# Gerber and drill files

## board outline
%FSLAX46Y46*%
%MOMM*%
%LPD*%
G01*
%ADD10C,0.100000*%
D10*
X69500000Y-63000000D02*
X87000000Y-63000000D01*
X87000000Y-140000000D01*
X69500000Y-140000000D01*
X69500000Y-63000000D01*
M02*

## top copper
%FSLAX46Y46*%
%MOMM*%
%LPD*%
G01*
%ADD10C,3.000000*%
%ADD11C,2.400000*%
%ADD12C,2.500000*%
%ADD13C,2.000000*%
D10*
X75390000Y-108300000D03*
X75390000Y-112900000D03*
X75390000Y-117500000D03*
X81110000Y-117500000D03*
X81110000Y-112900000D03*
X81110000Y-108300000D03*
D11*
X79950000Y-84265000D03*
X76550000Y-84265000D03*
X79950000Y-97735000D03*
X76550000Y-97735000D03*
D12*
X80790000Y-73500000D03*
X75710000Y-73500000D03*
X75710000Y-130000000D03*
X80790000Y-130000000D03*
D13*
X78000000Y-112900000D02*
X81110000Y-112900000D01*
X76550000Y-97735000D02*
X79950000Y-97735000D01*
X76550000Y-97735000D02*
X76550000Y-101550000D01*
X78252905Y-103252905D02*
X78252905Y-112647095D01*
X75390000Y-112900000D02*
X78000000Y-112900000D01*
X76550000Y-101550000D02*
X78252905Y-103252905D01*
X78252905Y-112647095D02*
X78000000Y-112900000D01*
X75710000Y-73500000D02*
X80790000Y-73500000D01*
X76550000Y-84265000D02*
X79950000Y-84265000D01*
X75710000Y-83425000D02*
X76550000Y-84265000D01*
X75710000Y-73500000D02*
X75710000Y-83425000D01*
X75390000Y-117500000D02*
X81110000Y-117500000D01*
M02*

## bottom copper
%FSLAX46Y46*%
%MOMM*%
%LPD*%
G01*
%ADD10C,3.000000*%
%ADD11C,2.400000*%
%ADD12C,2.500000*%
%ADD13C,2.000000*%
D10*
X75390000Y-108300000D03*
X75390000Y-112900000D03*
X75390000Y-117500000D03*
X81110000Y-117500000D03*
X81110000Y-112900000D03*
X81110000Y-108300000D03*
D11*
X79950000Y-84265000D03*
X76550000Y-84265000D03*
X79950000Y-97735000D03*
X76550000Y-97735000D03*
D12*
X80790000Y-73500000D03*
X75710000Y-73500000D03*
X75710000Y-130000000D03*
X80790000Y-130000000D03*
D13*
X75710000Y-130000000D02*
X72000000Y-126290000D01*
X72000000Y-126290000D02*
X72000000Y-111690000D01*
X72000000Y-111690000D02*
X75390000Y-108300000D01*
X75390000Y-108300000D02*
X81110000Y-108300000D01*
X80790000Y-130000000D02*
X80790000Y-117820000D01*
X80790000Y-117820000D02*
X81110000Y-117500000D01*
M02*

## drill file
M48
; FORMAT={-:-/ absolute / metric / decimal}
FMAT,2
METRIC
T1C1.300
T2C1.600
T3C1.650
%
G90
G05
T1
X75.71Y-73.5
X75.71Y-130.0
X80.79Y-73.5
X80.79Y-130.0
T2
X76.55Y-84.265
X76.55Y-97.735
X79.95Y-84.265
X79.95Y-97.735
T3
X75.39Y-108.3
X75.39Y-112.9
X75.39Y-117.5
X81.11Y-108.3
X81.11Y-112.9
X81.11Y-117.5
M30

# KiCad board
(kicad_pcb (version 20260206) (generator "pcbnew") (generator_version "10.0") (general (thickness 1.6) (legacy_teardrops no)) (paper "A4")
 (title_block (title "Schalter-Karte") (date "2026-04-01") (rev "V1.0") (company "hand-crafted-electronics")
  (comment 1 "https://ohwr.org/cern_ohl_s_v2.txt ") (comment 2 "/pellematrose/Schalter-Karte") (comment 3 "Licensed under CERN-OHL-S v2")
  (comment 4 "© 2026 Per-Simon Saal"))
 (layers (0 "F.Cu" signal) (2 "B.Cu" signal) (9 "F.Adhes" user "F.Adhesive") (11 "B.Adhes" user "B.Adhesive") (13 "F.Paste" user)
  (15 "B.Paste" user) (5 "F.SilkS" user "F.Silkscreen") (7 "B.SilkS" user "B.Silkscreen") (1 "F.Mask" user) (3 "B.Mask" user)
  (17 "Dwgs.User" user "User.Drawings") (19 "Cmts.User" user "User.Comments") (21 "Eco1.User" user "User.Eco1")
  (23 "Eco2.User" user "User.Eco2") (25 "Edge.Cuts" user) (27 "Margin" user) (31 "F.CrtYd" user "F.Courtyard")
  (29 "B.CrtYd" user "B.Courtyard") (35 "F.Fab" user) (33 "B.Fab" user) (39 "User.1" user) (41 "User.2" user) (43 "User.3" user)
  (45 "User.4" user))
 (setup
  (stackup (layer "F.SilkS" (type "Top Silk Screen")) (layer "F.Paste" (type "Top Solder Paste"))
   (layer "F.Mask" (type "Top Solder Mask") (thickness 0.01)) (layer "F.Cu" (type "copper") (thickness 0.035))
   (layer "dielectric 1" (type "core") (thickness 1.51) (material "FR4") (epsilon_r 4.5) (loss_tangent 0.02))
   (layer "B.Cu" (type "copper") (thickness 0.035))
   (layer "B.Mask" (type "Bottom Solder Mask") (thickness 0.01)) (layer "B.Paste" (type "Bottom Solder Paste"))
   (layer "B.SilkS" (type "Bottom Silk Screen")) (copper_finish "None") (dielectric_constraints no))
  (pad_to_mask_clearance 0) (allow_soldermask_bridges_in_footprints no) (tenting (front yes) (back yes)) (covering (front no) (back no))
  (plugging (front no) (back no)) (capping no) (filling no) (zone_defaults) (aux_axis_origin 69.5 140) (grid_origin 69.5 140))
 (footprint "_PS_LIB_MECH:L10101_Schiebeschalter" (layer "F.Cu") (at 78.25 112.9 90)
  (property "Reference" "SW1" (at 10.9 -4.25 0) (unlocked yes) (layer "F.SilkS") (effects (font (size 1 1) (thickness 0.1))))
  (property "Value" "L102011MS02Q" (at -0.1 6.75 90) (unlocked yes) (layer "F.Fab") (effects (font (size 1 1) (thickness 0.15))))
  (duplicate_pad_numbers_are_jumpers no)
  (pad "1" thru_hole circle (at 4.6 -2.86 90) (size 3 3) (drill 1.65) (layers "*.Cu" "*.Mask") (remove_unused_layers no)
   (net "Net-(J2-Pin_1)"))
  (pad "2" thru_hole circle (at 0 -2.86 90) (size 3 3) (drill 1.65) (layers "*.Cu" "*.Mask") (remove_unused_layers no) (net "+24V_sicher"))
  (pad "3" thru_hole circle (at -4.6 -2.86 90) (size 3 3) (drill 1.65) (layers "*.Cu" "*.Mask") (remove_unused_layers no)
   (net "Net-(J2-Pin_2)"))
  (pad "4" thru_hole circle (at -4.6 2.86 90) (size 3 3) (drill 1.65) (layers "*.Cu" "*.Mask") (remove_unused_layers no)
   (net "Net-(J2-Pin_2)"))
  (pad "5" thru_hole circle (at 0 2.86 90) (size 3 3) (drill 1.65) (layers "*.Cu" "*.Mask") (remove_unused_layers no) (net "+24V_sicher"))
  (pad "6" thru_hole circle (at 4.6 2.86 90) (size 3 3) (drill 1.65) (layers "*.Cu" "*.Mask") (remove_unused_layers no)
   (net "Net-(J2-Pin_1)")))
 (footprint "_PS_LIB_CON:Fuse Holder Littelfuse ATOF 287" (layer "F.Cu") (at 78.25 91 -90)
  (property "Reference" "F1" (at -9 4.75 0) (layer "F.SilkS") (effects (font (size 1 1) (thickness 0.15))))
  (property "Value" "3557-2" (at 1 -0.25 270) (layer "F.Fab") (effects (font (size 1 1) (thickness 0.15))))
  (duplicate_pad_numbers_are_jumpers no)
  (pad "1" thru_hole circle (at -6.735 -1.7 270) (size 2.4 2.4) (drill 1.6) (layers "*.Cu" "*.Mask") (remove_unused_layers no) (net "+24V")
   (solder_mask_margin 0.102))
  (pad "1" thru_hole circle (at -6.735 1.7 270) (size 2.4 2.4) (drill 1.6) (layers "*.Cu" "*.Mask") (remove_unused_layers no) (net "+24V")
   (solder_mask_margin 0.102))
  (pad "2" thru_hole circle (at 6.735 -1.7 270) (size 2.4 2.4) (drill 1.6) (layers "*.Cu" "*.Mask") (remove_unused_layers no)
   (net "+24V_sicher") (solder_mask_margin 0.102))
  (pad "2" thru_hole circle (at 6.735 1.7 270) (size 2.4 2.4) (drill 1.6) (layers "*.Cu" "*.Mask") (remove_unused_layers no)
   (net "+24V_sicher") (solder_mask_margin 0.102)))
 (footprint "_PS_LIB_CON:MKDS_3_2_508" (layer "F.Cu") (at 78.25 73.5 180)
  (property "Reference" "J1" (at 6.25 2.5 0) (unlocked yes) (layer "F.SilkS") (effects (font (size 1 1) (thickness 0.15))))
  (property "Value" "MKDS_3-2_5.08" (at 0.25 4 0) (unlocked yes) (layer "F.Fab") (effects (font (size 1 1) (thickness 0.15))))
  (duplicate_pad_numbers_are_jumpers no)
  (pad "1" thru_hole circle (at -2.54 0 180) (size 2.5 2.5) (drill 1.3) (layers "*.Cu" "*.Mask") (remove_unused_layers no) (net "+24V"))
  (pad "2" thru_hole circle (at 2.54 0 180) (size 2.5 2.5) (drill 1.3) (layers "*.Cu" "*.Mask") (remove_unused_layers no) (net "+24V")))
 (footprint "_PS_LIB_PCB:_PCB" (layer "F.Cu") (at 85.037731 101.98344 90)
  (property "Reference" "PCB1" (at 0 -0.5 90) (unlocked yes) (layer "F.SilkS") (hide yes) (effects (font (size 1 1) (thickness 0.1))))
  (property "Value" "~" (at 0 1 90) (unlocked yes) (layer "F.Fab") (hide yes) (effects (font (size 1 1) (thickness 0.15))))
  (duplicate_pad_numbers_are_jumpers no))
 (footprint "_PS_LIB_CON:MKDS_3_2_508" (layer "F.Cu") (at 78.25 130)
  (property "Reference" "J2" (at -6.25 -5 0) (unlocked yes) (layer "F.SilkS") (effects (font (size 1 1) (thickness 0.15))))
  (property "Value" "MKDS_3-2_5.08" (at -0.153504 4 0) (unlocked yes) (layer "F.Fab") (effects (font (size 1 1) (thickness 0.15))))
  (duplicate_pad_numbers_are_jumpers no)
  (pad "1" thru_hole circle (at -2.54 0) (size 2.5 2.5) (drill 1.3) (layers "*.Cu" "*.Mask") (remove_unused_layers no)
   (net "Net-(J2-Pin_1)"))
  (pad "2" thru_hole circle (at 2.54 0) (size 2.5 2.5) (drill 1.3) (layers "*.Cu" "*.Mask") (remove_unused_layers no) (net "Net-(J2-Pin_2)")))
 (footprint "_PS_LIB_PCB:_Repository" (layer "B.Cu") (at 85.300189 76.203735 -90)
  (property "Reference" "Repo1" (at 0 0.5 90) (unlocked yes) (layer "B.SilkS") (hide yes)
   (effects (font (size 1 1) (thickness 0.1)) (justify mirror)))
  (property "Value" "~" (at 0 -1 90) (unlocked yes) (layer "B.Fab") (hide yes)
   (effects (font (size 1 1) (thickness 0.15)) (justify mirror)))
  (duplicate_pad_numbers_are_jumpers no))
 (gr_rect (start 69.5 63) (end 87 140) (stroke (width 0.1) (type default)) (fill no) (layer "Edge.Cuts"))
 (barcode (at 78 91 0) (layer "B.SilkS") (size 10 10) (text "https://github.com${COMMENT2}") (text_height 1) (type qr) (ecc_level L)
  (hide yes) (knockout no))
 (segment (start 78 112.9) (end 81.11 112.9) (width 2) (layer "F.Cu") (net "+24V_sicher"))
 (segment (start 76.55 97.735) (end 79.95 97.735) (width 2) (layer "F.Cu") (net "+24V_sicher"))
 (segment (start 76.55 97.735) (end 76.55 101.55) (width 2) (layer "F.Cu") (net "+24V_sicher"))
 (segment (start 78.252905 103.252905) (end 78.252905 112.647095) (width 2) (layer "F.Cu") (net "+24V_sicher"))
 (segment (start 75.39 112.9) (end 78 112.9) (width 2) (layer "F.Cu") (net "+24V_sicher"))
 (segment (start 76.55 101.55) (end 78.252905 103.252905) (width 2) (layer "F.Cu") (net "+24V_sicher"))
 (segment (start 78.252905 112.647095) (end 78 112.9) (width 2) (layer "F.Cu") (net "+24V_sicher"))
 (segment (start 75.71 73.5) (end 80.79 73.5) (width 2) (layer "F.Cu") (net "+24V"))
 (segment (start 76.55 84.265) (end 79.95 84.265) (width 2) (layer "F.Cu") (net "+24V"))
 (segment (start 75.71 83.425) (end 76.55 84.265) (width 2) (layer "F.Cu") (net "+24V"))
 (segment (start 75.71 73.5) (end 75.71 83.425) (width 2) (layer "F.Cu") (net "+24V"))
 (segment (start 75.71 130) (end 72 126.29) (width 2) (layer "B.Cu") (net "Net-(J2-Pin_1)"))
 (segment (start 72 126.29) (end 72 111.69) (width 2) (layer "B.Cu") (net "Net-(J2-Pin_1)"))
 (segment (start 72 111.69) (end 75.39 108.3) (width 2) (layer "B.Cu") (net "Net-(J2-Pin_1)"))
 (segment (start 75.39 108.3) (end 81.11 108.3) (width 2) (layer "B.Cu") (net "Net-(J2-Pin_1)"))
 (segment (start 75.39 117.5) (end 81.11 117.5) (width 2) (layer "F.Cu") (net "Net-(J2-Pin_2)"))
 (segment (start 80.79 130) (end 80.79 117.82) (width 2) (layer "B.Cu") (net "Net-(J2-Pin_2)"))
 (segment (start 80.79 117.82) (end 81.11 117.5) (width 2) (layer "B.Cu") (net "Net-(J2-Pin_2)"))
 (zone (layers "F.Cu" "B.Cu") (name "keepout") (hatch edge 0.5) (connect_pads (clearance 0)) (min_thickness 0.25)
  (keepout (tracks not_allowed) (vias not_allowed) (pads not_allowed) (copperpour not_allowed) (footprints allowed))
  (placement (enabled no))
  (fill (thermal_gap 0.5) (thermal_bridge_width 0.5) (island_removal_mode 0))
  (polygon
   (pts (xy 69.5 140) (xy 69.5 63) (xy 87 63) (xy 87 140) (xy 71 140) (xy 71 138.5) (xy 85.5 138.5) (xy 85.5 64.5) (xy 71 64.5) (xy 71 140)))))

